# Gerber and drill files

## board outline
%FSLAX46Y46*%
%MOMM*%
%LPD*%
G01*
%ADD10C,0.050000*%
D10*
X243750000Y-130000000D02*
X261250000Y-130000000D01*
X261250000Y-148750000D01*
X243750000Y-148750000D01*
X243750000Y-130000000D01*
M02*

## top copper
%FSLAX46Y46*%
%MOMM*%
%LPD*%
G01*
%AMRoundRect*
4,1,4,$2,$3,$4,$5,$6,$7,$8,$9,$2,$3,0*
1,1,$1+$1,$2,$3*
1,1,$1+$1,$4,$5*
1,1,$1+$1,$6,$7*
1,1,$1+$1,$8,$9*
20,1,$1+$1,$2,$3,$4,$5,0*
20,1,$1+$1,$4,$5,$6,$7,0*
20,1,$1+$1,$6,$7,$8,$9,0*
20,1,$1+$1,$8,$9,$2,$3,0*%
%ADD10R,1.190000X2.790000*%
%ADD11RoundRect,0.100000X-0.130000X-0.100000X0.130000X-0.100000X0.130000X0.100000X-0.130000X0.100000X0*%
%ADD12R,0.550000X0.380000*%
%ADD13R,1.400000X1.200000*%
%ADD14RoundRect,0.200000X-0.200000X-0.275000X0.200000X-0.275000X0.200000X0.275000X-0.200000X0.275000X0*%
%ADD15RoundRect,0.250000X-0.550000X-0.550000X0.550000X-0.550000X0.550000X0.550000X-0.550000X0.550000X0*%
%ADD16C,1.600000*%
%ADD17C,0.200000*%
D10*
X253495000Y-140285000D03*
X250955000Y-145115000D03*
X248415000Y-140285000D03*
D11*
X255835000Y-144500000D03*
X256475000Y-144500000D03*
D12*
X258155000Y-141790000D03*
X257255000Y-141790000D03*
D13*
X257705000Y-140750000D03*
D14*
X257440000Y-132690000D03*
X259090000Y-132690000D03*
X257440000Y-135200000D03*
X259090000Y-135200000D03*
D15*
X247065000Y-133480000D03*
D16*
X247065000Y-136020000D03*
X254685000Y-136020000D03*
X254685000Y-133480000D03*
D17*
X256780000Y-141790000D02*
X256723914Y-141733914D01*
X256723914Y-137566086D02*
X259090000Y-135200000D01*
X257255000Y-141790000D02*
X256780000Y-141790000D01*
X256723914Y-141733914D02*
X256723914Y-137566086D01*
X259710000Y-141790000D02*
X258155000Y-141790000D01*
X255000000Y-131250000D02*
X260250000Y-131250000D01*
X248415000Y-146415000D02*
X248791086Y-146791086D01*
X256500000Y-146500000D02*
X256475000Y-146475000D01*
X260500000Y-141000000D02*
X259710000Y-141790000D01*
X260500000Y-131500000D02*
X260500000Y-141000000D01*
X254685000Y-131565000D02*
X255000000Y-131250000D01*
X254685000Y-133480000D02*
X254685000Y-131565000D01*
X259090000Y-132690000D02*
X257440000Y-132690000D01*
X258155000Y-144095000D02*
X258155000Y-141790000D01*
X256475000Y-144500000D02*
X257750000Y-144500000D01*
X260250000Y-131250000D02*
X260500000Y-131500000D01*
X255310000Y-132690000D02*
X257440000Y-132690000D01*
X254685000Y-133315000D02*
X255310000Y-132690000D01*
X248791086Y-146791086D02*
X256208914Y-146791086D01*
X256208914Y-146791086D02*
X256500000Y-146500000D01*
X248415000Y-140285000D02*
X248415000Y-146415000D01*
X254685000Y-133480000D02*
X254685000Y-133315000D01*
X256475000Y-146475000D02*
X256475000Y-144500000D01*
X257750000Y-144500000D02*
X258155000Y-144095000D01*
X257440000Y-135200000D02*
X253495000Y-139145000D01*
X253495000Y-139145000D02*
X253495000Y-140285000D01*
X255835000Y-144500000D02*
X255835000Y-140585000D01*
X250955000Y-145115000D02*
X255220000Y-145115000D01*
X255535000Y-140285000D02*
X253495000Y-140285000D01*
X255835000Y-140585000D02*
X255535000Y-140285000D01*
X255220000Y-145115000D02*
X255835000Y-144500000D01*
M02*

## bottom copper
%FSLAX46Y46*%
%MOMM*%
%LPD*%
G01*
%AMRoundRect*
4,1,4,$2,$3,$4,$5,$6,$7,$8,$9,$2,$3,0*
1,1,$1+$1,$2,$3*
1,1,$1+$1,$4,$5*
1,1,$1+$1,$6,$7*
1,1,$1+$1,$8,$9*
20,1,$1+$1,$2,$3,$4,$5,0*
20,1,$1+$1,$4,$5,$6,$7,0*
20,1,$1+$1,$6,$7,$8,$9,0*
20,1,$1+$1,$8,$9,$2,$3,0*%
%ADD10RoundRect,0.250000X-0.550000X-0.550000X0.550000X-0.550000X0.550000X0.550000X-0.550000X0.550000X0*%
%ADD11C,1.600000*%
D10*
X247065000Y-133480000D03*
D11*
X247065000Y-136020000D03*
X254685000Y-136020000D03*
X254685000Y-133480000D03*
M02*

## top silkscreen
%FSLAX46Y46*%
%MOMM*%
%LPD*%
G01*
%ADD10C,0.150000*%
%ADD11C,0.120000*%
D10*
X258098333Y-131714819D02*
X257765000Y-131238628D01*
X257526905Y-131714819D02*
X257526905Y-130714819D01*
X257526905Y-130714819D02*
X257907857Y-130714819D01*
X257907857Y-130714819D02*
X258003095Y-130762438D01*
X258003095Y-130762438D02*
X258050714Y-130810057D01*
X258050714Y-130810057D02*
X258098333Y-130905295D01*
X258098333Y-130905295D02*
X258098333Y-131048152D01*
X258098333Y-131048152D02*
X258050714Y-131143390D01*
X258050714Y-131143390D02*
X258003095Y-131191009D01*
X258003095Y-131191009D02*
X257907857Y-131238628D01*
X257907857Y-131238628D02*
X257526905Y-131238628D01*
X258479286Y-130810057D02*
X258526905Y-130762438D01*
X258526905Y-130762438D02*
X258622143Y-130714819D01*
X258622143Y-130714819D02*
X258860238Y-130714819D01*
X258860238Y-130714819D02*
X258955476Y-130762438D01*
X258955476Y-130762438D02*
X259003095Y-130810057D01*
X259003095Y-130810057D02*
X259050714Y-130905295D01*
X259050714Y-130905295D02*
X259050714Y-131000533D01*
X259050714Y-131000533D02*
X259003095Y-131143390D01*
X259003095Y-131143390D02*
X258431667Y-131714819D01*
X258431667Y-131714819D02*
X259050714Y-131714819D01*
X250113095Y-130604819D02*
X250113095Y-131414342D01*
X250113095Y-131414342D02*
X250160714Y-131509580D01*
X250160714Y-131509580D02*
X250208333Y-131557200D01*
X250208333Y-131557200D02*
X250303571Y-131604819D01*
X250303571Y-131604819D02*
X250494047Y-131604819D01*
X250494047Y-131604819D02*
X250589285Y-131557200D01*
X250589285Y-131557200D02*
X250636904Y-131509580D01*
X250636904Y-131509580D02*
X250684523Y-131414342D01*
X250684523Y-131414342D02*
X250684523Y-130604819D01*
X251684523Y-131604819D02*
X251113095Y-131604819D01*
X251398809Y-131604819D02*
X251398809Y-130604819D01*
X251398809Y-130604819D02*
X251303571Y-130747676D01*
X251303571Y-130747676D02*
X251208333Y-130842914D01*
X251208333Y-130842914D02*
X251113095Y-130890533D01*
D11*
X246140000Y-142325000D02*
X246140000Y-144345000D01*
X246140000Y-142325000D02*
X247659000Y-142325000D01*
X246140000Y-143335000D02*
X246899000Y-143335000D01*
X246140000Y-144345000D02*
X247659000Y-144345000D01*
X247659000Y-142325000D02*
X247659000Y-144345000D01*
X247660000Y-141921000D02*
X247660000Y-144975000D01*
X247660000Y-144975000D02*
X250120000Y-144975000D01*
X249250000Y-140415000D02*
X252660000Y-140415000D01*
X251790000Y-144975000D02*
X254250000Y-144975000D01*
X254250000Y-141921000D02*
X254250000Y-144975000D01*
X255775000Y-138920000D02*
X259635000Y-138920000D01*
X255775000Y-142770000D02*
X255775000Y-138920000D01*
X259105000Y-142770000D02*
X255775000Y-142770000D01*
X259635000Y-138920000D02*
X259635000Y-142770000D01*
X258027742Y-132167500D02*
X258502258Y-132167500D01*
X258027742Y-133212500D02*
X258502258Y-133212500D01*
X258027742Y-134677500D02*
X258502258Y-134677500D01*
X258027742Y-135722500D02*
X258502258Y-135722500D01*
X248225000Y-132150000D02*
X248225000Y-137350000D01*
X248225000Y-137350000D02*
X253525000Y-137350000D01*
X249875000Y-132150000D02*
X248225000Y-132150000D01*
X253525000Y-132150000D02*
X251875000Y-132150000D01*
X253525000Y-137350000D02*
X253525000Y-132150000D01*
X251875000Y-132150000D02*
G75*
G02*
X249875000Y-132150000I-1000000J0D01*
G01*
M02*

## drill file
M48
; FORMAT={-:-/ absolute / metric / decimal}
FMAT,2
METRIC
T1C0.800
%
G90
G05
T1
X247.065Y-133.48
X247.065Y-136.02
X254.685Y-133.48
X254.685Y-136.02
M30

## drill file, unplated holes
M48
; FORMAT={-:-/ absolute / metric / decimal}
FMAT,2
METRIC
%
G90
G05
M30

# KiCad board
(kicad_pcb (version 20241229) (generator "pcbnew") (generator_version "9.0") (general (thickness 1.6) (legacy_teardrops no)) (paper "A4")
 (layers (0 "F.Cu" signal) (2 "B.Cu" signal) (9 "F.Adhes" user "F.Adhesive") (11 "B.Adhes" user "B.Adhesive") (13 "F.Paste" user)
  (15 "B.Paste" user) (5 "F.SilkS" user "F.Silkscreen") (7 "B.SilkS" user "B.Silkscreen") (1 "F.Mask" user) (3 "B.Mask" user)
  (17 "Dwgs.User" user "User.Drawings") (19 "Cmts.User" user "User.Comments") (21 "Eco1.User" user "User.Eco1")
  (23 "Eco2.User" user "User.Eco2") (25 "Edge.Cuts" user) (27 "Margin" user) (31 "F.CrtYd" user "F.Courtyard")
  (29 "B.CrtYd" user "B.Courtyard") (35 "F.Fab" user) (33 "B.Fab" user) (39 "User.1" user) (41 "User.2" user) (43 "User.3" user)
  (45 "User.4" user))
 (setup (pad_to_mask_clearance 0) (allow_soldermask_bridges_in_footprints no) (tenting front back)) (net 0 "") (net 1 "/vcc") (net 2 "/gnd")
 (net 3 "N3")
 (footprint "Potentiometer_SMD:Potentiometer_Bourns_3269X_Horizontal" (layer "F.Cu") (at 250.955 142.7)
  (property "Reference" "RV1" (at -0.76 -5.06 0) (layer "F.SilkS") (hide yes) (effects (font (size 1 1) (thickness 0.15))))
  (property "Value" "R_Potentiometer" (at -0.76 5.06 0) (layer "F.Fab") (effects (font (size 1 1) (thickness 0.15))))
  (fp_line (start -4.815 -0.375) (end -4.815 1.645) (stroke (width 0.12) (type solid)) (layer "F.SilkS"))
  (fp_line (start -4.815 -0.375) (end -3.296 -0.375) (stroke (width 0.12) (type solid)) (layer "F.SilkS"))
  (fp_line (start -4.815 0.635) (end -4.056 0.635) (stroke (width 0.12) (type solid)) (layer "F.SilkS"))
  (fp_line (start -4.815 1.645) (end -3.296 1.645) (stroke (width 0.12) (type solid)) (layer "F.SilkS"))
  (fp_line (start -3.296 -0.375) (end -3.296 1.645) (stroke (width 0.12) (type solid)) (layer "F.SilkS"))
  (fp_line (start -3.295 -0.779) (end -3.295 2.275) (stroke (width 0.12) (type solid)) (layer "F.SilkS"))
  (fp_line (start -3.295 2.275) (end -0.835 2.275) (stroke (width 0.12) (type solid)) (layer "F.SilkS"))
  (fp_line (start -1.705 -2.285) (end 1.705 -2.285) (stroke (width 0.12) (type solid)) (layer "F.SilkS"))
  (fp_line (start 0.835 2.275) (end 3.295 2.275) (stroke (width 0.12) (type solid)) (layer "F.SilkS"))
  (fp_line (start 3.295 -0.779) (end 3.295 2.275) (stroke (width 0.12) (type solid)) (layer "F.SilkS"))
  (pad "1" smd rect (at 2.54 -2.415) (size 1.19 2.79) (layers "F.Cu" "F.Mask" "F.Paste") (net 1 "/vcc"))
  (pad "2" smd rect (at 0 2.415) (size 1.19 2.79) (layers "F.Cu" "F.Mask" "F.Paste") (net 1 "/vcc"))
  (pad "3" smd rect (at -2.54 -2.415) (size 1.19 2.79) (layers "F.Cu" "F.Mask" "F.Paste") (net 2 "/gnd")))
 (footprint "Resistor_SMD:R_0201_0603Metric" (layer "F.Cu") (at 256.155 144.5)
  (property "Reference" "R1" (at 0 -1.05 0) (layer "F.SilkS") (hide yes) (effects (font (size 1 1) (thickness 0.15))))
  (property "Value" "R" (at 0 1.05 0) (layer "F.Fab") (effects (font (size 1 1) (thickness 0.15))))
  (pad "" smd roundrect (at -0.345 0) (size 0.318 0.36) (layers "F.Paste") (roundrect_rratio 0.25))
  (pad "" smd roundrect (at 0.345 0) (size 0.318 0.36) (layers "F.Paste") (roundrect_rratio 0.25))
  (pad "1" smd roundrect (at -0.32 0) (size 0.46 0.4) (layers "F.Cu" "F.Mask") (roundrect_rratio 0.25) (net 1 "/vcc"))
  (pad "2" smd roundrect (at 0.32 0) (size 0.46 0.4) (layers "F.Cu" "F.Mask") (roundrect_rratio 0.25) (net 2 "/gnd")))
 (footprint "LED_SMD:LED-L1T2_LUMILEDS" (layer "F.Cu") (at 257.705 141.27)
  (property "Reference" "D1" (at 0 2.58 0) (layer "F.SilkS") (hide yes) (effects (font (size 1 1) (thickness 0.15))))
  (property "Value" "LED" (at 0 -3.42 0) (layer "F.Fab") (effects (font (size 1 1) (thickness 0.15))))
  (fp_line (start -1.93 -2.35) (end 1.93 -2.35) (stroke (width 0.12) (type solid)) (layer "F.SilkS"))
  (fp_line (start -1.93 1.5) (end -1.93 -2.35) (stroke (width 0.12) (type solid)) (layer "F.SilkS"))
  (fp_line (start 1.4 1.5) (end -1.93 1.5) (stroke (width 0.12) (type solid)) (layer "F.SilkS"))
  (fp_line (start 1.93 -2.35) (end 1.93 1.5) (stroke (width 0.12) (type solid)) (layer "F.SilkS"))
  (pad "1" smd rect (at 0.45 0.52) (size 0.55 0.38) (layers "F.Cu" "F.Mask" "F.Paste") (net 2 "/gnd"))
  (pad "2" smd rect (at -0.45 0.52) (size 0.55 0.38) (layers "F.Cu" "F.Mask" "F.Paste") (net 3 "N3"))
  (pad "3" smd rect (at 0 -0.52) (size 1.4 1.2) (layers "F.Cu" "F.Mask" "F.Paste")))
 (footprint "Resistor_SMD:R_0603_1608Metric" (layer "F.Cu") (at 258.265 132.69)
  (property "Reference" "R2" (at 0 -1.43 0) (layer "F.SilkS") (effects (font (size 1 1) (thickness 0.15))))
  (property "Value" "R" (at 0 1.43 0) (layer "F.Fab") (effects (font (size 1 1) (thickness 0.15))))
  (fp_line (start -0.237258 -0.5225) (end 0.237258 -0.5225) (stroke (width 0.12) (type solid)) (layer "F.SilkS"))
  (fp_line (start -0.237258 0.5225) (end 0.237258 0.5225) (stroke (width 0.12) (type solid)) (layer "F.SilkS"))
  (pad "1" smd roundrect (at -0.825 0) (size 0.8 0.95) (layers "F.Cu" "F.Mask" "F.Paste") (roundrect_rratio 0.25) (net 2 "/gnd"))
  (pad "2" smd roundrect (at 0.825 0) (size 0.8 0.95) (layers "F.Cu" "F.Mask" "F.Paste") (roundrect_rratio 0.25) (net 2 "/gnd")))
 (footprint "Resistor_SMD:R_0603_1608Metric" (layer "F.Cu") (at 258.265 135.2)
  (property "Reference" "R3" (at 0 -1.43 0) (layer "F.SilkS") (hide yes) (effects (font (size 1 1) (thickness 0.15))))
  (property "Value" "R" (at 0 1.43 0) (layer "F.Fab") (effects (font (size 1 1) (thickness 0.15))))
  (fp_line (start -0.237258 -0.5225) (end 0.237258 -0.5225) (stroke (width 0.12) (type solid)) (layer "F.SilkS"))
  (fp_line (start -0.237258 0.5225) (end 0.237258 0.5225) (stroke (width 0.12) (type solid)) (layer "F.SilkS"))
  (pad "1" smd roundrect (at -0.825 0) (size 0.8 0.95) (layers "F.Cu" "F.Mask" "F.Paste") (roundrect_rratio 0.25) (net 1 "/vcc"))
  (pad "2" smd roundrect (at 0.825 0) (size 0.8 0.95) (layers "F.Cu" "F.Mask" "F.Paste") (roundrect_rratio 0.25) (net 3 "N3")))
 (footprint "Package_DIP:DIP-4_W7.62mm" (layer "F.Cu") (at 247.065 133.48)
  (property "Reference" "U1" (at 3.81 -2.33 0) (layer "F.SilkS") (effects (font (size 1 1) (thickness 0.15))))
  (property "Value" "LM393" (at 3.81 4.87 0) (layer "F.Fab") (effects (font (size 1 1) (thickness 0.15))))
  (fp_line (start 1.16 -1.33) (end 1.16 3.87) (stroke (width 0.12) (type solid)) (layer "F.SilkS"))
  (fp_line (start 1.16 3.87) (end 6.46 3.87) (stroke (width 0.12) (type solid)) (layer "F.SilkS"))
  (fp_line (start 2.81 -1.33) (end 1.16 -1.33) (stroke (width 0.12) (type solid)) (layer "F.SilkS"))
  (fp_line (start 6.46 -1.33) (end 4.81 -1.33) (stroke (width 0.12) (type solid)) (layer "F.SilkS"))
  (fp_line (start 6.46 3.87) (end 6.46 -1.33) (stroke (width 0.12) (type solid)) (layer "F.SilkS"))
  (fp_arc (start 4.81 -1.33) (mid 3.81 -0.33) (end 2.81 -1.33) (stroke (width 0.12) (type solid)) (layer "F.SilkS"))
  (pad "1" thru_hole roundrect (at 0 0) (size 1.6 1.6) (drill 0.8) (layers "*.Cu" "*.Mask") (remove_unused_layers no)
   (roundrect_rratio 0.15625))
  (pad "2" thru_hole circle (at 0 2.54) (size 1.6 1.6) (drill 0.8) (layers "*.Cu" "*.Mask") (remove_unused_layers no))
  (pad "3" thru_hole circle (at 7.62 2.54) (size 1.6 1.6) (drill 0.8) (layers "*.Cu" "*.Mask") (remove_unused_layers no))
  (pad "4" thru_hole circle (at 7.62 0) (size 1.6 1.6) (drill 0.8) (layers "*.Cu" "*.Mask") (remove_unused_layers no) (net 2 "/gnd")))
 (gr_rect (start 243.75 130) (end 261.25 148.75) (stroke (width 0.05) (type default)) (fill no) (layer "Edge.Cuts"))
 (segment (start 256.78 141.79) (end 256.723914 141.733914) (width 0.2) (layer "F.Cu") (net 3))
 (segment (start 256.723914 137.566086) (end 259.09 135.2) (width 0.2) (layer "F.Cu") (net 3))
 (segment (start 257.255 141.79) (end 256.78 141.79) (width 0.2) (layer "F.Cu") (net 3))
 (segment (start 256.723914 141.733914) (end 256.723914 137.566086) (width 0.2) (layer "F.Cu") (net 3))
 (segment (start 259.71 141.79) (end 258.155 141.79) (width 0.2) (layer "F.Cu") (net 2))
 (segment (start 255 131.25) (end 260.25 131.25) (width 0.2) (layer "F.Cu") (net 2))
 (segment (start 248.415 146.415) (end 248.791086 146.791086) (width 0.2) (layer "F.Cu") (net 2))
 (segment (start 256.5 146.5) (end 256.475 146.475) (width 0.2) (layer "F.Cu") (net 2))
 (segment (start 260.5 141) (end 259.71 141.79) (width 0.2) (layer "F.Cu") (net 2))
 (segment (start 260.5 131.5) (end 260.5 141) (width 0.2) (layer "F.Cu") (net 2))
 (segment (start 254.685 131.565) (end 255 131.25) (width 0.2) (layer "F.Cu") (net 2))
 (segment (start 254.685 133.48) (end 254.685 131.565) (width 0.2) (layer "F.Cu") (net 2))
 (segment (start 259.09 132.69) (end 257.44 132.69) (width 0.2) (layer "F.Cu") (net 2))
 (segment (start 258.155 144.095) (end 258.155 141.79) (width 0.2) (layer "F.Cu") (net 2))
 (segment (start 256.475 144.5) (end 257.75 144.5) (width 0.2) (layer "F.Cu") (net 2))
 (segment (start 260.25 131.25) (end 260.5 131.5) (width 0.2) (layer "F.Cu") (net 2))
 (segment (start 255.31 132.69) (end 257.44 132.69) (width 0.2) (layer "F.Cu") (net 2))
 (segment (start 254.685 133.315) (end 255.31 132.69) (width 0.2) (layer "F.Cu") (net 2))
 (segment (start 248.791086 146.791086) (end 256.208914 146.791086) (width 0.2) (layer "F.Cu") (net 2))
 (segment (start 256.208914 146.791086) (end 256.5 146.5) (width 0.2) (layer "F.Cu") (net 2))
 (segment (start 248.415 140.285) (end 248.415 146.415) (width 0.2) (layer "F.Cu") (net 2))
 (segment (start 254.685 133.48) (end 254.685 133.315) (width 0.2) (layer "F.Cu") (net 2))
 (segment (start 256.475 146.475) (end 256.475 144.5) (width 0.2) (layer "F.Cu") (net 2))
 (segment (start 257.75 144.5) (end 258.155 144.095) (width 0.2) (layer "F.Cu") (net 2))
 (segment (start 257.44 135.2) (end 253.495 139.145) (width 0.2) (layer "F.Cu") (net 1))
 (segment (start 253.495 139.145) (end 253.495 140.285) (width 0.2) (layer "F.Cu") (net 1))
 (segment (start 255.835 144.5) (end 255.835 140.585) (width 0.2) (layer "F.Cu") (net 1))
 (segment (start 250.955 145.115) (end 255.22 145.115) (width 0.2) (layer "F.Cu") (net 1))
 (segment (start 255.535 140.285) (end 253.495 140.285) (width 0.2) (layer "F.Cu") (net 1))
 (segment (start 255.835 140.585) (end 255.535 140.285) (width 0.2) (layer "F.Cu") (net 1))
 (segment (start 255.22 145.115) (end 255.835 144.5) (width 0.2) (layer "F.Cu") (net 1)))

